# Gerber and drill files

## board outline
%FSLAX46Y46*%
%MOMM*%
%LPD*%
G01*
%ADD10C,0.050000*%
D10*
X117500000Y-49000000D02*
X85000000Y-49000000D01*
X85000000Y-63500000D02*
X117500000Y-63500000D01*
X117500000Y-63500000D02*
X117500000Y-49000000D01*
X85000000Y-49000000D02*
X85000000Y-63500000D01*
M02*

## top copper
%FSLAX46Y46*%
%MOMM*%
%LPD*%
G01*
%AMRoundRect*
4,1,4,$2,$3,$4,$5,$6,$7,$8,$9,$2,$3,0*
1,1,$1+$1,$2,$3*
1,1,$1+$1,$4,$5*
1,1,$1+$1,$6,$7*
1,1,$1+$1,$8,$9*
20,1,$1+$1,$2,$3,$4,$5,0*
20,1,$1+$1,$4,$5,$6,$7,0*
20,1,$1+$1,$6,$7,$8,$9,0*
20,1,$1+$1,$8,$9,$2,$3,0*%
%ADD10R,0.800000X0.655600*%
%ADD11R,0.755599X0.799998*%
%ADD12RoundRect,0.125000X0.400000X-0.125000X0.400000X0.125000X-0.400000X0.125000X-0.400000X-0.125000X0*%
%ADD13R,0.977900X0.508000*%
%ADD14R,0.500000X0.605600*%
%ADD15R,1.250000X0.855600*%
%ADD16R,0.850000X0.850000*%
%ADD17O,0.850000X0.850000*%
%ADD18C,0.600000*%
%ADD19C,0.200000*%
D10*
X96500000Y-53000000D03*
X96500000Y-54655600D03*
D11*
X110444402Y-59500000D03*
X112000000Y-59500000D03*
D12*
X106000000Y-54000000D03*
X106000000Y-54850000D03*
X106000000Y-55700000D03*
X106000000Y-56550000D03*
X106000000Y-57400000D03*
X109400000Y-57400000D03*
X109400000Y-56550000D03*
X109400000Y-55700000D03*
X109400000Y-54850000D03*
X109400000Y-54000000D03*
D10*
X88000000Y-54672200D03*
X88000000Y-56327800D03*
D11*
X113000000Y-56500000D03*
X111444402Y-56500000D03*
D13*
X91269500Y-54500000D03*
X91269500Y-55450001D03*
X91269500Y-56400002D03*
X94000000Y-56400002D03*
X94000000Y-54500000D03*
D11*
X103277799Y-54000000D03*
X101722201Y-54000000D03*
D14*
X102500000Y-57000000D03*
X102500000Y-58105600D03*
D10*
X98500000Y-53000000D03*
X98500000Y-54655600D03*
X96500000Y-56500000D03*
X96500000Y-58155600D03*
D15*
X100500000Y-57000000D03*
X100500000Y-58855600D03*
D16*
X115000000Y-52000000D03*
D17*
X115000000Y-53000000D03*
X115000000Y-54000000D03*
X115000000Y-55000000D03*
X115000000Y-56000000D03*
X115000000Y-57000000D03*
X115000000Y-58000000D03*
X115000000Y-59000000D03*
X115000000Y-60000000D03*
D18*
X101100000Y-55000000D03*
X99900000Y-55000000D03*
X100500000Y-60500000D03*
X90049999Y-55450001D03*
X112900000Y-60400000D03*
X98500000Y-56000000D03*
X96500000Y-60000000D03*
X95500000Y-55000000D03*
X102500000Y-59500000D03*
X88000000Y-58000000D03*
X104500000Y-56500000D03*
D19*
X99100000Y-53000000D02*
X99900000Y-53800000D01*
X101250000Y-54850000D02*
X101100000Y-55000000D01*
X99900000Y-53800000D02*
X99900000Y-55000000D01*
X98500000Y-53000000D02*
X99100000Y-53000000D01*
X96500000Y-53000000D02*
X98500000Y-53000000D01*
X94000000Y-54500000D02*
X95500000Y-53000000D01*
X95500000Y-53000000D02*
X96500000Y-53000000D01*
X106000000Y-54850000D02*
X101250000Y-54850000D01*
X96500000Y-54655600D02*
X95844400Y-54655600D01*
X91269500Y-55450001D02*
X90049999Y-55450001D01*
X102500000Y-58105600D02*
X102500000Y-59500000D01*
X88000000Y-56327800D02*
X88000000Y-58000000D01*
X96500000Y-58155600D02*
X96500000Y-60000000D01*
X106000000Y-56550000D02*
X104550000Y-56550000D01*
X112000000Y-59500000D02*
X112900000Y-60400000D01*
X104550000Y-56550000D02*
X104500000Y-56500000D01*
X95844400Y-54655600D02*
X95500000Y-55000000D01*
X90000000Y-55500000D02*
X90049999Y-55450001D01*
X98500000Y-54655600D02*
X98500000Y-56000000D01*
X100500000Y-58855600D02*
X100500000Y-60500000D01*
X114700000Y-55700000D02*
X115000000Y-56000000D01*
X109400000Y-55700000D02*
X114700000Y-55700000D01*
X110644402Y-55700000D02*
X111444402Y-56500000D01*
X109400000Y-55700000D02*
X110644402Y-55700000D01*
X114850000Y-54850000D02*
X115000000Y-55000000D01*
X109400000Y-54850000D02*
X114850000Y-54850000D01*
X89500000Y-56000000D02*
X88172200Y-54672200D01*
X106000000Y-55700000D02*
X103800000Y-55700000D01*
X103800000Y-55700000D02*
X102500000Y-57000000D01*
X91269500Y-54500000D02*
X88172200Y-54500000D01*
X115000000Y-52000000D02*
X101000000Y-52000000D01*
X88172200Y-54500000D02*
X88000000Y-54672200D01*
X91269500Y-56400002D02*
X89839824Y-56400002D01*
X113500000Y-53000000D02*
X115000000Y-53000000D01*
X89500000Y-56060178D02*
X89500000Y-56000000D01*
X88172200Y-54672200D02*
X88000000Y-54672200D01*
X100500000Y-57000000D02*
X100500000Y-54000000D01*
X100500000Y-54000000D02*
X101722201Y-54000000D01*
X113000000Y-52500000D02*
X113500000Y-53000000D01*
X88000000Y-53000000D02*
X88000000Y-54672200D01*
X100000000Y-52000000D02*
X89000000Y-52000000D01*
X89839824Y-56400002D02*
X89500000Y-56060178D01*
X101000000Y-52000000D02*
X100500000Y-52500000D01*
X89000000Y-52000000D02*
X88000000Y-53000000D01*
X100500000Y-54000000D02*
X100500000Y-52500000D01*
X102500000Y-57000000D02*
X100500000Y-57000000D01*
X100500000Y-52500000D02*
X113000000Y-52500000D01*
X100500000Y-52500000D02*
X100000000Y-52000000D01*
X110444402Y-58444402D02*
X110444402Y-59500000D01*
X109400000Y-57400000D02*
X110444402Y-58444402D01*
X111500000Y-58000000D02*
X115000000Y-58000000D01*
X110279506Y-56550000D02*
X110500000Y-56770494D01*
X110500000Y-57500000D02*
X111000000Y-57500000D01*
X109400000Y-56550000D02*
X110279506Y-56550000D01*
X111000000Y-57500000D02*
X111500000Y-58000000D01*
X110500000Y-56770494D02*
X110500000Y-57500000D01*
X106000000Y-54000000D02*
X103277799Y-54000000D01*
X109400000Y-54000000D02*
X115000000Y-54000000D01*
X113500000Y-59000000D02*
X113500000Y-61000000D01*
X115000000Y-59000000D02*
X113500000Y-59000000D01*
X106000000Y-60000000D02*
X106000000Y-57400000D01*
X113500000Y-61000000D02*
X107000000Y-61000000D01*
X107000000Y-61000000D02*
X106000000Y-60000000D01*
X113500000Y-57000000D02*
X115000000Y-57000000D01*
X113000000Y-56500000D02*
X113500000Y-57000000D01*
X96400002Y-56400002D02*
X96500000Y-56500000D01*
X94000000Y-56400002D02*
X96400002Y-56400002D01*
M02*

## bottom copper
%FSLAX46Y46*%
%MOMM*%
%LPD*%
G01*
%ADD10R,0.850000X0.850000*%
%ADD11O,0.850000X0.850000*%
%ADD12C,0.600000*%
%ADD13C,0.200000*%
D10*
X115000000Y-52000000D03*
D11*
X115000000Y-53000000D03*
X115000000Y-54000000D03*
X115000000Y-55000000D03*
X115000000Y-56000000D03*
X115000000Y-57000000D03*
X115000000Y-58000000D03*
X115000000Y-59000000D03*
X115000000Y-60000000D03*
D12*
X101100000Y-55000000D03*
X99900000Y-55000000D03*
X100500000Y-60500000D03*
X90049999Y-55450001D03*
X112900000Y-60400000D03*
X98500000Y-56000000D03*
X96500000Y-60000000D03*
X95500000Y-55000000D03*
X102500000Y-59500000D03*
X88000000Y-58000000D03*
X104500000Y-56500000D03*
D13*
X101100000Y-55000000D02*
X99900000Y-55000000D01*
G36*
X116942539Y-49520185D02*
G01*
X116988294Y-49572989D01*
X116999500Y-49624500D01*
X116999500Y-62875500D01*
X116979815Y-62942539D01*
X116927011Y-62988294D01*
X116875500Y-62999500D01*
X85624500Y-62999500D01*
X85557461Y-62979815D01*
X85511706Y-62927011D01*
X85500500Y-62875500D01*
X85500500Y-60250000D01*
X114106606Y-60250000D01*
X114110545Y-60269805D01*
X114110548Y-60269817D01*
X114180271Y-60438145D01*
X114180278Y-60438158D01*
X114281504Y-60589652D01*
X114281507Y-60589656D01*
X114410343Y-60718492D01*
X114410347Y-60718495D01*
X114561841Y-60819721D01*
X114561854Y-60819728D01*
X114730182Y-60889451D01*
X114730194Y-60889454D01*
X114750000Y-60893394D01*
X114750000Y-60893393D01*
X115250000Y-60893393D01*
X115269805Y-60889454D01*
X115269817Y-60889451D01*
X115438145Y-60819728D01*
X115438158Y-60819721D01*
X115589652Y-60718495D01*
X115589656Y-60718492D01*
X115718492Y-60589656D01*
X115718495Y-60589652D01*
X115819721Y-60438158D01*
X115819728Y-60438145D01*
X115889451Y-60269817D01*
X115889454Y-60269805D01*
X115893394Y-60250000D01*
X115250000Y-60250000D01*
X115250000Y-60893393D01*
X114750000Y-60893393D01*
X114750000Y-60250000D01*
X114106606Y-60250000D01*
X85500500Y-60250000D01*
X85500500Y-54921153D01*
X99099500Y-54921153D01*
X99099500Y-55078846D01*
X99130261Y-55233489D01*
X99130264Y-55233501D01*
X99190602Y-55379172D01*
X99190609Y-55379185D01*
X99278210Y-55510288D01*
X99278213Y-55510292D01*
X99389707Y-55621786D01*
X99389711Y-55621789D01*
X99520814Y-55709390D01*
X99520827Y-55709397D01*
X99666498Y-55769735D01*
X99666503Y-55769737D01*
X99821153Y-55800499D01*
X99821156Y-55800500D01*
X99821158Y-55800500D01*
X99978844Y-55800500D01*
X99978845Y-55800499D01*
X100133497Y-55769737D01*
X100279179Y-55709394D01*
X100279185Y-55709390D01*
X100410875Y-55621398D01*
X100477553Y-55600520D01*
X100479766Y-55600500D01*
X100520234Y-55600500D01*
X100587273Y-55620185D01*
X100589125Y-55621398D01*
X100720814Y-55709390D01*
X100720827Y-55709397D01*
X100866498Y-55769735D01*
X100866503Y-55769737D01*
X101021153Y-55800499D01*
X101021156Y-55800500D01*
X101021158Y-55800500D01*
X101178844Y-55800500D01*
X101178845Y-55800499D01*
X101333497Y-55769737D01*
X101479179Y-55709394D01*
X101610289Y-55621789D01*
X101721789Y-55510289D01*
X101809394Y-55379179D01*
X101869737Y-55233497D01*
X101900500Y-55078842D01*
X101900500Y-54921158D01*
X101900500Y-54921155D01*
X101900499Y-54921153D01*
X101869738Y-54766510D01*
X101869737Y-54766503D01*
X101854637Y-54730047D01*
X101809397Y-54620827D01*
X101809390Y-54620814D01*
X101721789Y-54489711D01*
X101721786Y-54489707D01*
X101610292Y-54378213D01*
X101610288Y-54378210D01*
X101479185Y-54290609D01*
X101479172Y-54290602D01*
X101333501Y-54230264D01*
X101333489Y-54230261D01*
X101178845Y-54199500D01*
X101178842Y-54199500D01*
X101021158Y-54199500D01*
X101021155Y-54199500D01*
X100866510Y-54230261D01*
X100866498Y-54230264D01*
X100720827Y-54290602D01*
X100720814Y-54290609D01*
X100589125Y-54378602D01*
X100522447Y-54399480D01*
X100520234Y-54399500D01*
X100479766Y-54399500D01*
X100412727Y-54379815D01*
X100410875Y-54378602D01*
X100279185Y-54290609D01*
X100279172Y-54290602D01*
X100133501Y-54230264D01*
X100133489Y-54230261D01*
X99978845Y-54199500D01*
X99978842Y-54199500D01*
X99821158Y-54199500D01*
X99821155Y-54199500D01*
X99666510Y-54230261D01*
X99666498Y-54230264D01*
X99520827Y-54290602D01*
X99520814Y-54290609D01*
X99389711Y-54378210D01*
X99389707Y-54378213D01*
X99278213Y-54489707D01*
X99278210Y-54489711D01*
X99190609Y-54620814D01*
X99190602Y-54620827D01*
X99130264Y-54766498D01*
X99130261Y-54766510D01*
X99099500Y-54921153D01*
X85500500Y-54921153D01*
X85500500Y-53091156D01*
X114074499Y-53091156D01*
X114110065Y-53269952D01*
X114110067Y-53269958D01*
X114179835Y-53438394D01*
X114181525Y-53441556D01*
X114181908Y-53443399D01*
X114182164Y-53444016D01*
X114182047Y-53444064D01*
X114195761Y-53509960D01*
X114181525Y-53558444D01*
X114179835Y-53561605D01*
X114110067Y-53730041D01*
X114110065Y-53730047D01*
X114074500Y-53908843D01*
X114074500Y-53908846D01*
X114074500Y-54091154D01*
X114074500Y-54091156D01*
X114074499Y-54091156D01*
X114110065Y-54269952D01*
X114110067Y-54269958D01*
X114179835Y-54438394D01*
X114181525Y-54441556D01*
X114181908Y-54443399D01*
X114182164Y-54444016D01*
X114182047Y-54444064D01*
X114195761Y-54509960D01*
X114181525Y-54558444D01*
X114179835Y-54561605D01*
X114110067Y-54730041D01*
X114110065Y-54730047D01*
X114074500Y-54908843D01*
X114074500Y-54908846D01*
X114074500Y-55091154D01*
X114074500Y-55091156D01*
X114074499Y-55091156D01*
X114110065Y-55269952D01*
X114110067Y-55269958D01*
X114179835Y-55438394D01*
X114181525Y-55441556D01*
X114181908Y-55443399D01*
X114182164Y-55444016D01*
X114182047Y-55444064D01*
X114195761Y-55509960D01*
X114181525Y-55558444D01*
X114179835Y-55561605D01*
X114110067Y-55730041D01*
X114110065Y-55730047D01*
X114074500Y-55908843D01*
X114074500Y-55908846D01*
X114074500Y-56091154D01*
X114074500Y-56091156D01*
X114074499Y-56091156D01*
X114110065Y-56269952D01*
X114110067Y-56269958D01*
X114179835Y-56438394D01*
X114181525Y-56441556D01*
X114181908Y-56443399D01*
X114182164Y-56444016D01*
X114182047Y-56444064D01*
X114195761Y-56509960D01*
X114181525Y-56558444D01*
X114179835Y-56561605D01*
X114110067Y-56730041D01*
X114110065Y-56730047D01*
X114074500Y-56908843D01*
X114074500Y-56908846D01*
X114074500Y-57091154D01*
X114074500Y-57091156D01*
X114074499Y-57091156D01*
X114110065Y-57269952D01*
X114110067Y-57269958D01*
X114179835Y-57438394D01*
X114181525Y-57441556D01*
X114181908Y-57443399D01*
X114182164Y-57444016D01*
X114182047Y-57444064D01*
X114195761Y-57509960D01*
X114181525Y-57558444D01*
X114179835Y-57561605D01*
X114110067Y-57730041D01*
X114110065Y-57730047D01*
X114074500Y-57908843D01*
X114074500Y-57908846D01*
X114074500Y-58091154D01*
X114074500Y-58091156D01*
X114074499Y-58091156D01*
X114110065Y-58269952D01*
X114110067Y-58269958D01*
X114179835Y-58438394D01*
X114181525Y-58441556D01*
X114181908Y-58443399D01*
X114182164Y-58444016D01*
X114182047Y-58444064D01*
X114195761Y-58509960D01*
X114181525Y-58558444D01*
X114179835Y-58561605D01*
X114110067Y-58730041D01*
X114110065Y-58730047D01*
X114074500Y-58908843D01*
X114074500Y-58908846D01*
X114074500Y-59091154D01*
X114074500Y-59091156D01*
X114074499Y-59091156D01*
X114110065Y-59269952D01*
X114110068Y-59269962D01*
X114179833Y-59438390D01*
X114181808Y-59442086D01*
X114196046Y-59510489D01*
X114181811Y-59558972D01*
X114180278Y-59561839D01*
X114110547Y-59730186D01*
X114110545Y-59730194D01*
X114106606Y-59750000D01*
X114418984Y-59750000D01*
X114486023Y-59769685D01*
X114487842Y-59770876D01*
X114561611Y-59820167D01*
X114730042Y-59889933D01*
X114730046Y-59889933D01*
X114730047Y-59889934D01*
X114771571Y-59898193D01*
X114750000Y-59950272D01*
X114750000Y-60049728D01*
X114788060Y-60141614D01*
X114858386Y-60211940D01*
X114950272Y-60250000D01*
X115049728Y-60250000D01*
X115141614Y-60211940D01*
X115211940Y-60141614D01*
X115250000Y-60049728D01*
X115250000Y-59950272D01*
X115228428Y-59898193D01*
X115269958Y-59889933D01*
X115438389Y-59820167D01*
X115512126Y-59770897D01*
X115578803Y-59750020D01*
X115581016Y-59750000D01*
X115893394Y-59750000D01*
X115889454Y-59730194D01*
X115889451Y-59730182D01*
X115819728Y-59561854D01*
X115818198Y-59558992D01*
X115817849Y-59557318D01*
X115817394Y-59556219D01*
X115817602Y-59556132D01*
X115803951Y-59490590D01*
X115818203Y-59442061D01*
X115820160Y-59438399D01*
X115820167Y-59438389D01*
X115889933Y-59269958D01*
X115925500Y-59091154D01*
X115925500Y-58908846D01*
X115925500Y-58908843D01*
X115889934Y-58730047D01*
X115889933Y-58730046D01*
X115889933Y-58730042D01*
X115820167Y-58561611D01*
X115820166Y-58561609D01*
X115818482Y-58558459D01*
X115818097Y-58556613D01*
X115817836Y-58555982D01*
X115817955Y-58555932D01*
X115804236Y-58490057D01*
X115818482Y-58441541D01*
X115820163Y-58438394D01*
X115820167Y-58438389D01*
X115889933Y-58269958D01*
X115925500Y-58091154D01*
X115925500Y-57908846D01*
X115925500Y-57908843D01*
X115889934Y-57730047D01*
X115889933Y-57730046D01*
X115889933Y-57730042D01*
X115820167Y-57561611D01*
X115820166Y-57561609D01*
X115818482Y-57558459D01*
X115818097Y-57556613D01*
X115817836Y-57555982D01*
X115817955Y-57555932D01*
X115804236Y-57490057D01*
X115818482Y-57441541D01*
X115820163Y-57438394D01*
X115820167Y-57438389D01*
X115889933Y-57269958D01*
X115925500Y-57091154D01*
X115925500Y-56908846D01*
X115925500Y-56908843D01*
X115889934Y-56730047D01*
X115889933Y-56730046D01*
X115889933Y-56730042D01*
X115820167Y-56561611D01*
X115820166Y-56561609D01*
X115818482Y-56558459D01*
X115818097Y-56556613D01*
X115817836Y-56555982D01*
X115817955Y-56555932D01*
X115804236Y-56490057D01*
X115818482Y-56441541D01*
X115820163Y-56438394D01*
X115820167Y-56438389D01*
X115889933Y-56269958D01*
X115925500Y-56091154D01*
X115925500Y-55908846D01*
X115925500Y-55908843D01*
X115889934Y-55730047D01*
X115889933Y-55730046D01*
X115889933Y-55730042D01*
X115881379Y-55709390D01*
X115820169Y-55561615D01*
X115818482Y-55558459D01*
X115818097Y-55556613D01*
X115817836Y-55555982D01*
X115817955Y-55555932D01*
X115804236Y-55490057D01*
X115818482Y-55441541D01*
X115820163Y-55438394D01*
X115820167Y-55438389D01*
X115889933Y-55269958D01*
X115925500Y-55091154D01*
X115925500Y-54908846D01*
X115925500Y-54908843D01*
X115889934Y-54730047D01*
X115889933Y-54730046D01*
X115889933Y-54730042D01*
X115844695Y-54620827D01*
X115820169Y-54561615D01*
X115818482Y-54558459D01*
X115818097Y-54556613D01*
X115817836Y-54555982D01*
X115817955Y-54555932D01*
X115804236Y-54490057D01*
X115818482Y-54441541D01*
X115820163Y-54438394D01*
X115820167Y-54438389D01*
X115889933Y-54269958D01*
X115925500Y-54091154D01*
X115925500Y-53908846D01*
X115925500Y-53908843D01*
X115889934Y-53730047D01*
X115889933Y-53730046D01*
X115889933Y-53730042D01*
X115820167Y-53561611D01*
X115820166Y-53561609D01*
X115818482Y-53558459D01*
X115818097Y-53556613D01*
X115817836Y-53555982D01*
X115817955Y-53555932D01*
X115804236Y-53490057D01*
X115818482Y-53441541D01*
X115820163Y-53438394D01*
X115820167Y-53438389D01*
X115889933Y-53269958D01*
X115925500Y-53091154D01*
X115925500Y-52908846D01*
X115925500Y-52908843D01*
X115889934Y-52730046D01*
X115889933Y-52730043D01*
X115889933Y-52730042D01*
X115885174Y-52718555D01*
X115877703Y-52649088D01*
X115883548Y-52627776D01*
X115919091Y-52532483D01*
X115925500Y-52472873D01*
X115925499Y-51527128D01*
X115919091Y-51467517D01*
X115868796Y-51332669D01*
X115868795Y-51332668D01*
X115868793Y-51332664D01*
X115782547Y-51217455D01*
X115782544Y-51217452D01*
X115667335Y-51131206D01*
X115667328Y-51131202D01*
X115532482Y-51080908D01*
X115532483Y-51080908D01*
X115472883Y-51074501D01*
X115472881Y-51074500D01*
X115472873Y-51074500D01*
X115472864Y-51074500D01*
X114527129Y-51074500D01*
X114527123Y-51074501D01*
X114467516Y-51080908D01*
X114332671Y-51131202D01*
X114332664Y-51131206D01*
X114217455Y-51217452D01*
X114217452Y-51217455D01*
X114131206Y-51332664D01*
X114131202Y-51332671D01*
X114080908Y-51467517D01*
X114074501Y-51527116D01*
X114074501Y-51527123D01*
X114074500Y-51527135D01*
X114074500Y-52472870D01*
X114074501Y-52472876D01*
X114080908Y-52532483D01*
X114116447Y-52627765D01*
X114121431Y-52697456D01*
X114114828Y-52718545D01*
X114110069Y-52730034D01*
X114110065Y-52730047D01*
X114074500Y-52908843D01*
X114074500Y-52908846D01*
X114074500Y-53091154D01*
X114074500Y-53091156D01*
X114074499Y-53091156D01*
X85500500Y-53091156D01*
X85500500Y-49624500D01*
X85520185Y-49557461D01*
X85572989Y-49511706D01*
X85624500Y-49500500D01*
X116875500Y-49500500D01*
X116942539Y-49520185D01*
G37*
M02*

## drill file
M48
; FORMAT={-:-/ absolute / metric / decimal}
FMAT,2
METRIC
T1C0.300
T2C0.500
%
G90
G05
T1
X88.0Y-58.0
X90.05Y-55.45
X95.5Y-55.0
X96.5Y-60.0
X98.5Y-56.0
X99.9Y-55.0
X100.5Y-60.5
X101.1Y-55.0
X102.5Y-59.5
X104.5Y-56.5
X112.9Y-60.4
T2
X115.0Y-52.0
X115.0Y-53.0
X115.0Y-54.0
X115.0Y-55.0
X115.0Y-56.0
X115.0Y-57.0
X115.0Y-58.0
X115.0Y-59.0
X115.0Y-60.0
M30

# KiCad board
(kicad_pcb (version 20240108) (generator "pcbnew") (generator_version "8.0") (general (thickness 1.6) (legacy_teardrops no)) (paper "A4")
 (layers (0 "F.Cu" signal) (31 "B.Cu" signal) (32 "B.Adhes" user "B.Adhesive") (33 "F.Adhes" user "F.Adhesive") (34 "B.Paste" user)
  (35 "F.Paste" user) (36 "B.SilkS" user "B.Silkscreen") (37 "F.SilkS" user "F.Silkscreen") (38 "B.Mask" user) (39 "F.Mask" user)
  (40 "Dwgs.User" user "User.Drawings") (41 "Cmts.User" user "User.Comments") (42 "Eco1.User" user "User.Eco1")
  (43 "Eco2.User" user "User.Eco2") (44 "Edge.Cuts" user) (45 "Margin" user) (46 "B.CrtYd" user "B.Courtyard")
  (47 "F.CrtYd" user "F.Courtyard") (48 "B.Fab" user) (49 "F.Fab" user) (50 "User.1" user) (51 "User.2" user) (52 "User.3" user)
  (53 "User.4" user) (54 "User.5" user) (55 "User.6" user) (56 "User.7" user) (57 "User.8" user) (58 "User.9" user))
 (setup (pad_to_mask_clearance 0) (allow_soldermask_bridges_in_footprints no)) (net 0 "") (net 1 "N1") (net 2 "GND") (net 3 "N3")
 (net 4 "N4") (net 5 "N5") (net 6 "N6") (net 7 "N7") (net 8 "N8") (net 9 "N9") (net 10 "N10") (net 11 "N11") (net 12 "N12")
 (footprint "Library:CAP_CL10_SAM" (layer "F.Cu") (at 96.5 53.8278 -90)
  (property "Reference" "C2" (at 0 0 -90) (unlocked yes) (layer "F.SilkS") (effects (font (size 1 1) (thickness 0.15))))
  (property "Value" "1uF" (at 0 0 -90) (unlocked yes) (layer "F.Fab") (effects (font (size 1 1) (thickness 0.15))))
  (pad "1" smd rect (at -0.8278 0 270) (size 0.6556 0.8) (layers "F.Cu" "F.Paste" "F.Mask") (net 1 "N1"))
  (pad "2" smd rect (at 0.8278 0 270) (size 0.6556 0.8) (layers "F.Cu" "F.Paste" "F.Mask") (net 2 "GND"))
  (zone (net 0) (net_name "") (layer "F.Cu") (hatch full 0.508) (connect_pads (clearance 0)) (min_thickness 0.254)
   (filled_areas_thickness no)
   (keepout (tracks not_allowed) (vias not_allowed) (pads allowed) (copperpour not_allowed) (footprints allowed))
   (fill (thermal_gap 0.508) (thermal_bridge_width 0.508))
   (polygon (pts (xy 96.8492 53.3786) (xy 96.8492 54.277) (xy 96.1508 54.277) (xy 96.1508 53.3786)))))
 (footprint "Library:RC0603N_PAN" (layer "F.Cu") (at 111.222201 59.5)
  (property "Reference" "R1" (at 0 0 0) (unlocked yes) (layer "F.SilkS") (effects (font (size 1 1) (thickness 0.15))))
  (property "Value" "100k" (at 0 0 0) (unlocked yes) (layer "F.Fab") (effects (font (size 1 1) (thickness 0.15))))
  (pad "1" smd rect (at -0.777799 0) (size 0.755599 0.799998) (layers "F.Cu" "F.Paste" "F.Mask") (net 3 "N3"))
  (pad "2" smd rect (at 0.777799 0) (size 0.755599 0.799998) (layers "F.Cu" "F.Paste" "F.Mask") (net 2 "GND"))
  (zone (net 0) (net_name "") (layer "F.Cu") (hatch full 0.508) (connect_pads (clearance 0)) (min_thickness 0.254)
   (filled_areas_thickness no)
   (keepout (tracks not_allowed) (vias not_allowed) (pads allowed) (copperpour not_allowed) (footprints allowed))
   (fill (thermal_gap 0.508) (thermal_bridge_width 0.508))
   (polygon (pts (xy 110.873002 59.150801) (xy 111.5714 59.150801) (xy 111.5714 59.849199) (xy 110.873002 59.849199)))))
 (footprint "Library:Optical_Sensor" (layer "F.Cu") (at 116.5 60.5)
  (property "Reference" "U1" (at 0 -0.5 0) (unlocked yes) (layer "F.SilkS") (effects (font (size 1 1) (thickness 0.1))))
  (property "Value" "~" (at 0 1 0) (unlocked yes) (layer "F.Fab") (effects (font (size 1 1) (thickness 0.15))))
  (pad "1" smd roundrect (at -10.5 -6.5 90) (size 0.5 1.05) (layers "F.Cu" "F.Paste" "F.Mask") (roundrect_rratio 0.25) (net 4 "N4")
   (thermal_bridge_angle 45))
  (pad "2" smd roundrect (at -10.5 -5.65 90) (size 0.5 1.05) (layers "F.Cu" "F.Paste" "F.Mask") (roundrect_rratio 0.25) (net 1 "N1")
   (thermal_bridge_angle 45))
  (pad "3" smd roundrect (at -10.5 -4.8 90) (size 0.5 1.05) (layers "F.Cu" "F.Paste" "F.Mask") (roundrect_rratio 0.25) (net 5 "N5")
   (thermal_bridge_angle 45))
  (pad "4" smd roundrect (at -10.5 -3.95 90) (size 0.5 1.05) (layers "F.Cu" "F.Paste" "F.Mask") (roundrect_rratio 0.25) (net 2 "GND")
   (thermal_bridge_angle 45))
  (pad "5" smd roundrect (at -10.5 -3.1 90) (size 0.5 1.05) (layers "F.Cu" "F.Paste" "F.Mask") (roundrect_rratio 0.25) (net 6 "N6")
   (thermal_bridge_angle 45))
  (pad "6" smd roundrect (at -7.1 -3.1 90) (size 0.5 1.05) (layers "F.Cu" "F.Paste" "F.Mask") (roundrect_rratio 0.25) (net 3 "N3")
   (thermal_bridge_angle 45))
  (pad "7" smd roundrect (at -7.1 -3.95 90) (size 0.5 1.05) (layers "F.Cu" "F.Paste" "F.Mask") (roundrect_rratio 0.25) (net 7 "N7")
   (thermal_bridge_angle 45))
  (pad "8" smd roundrect (at -7.1 -4.8 90) (size 0.5 1.05) (layers "F.Cu" "F.Paste" "F.Mask") (roundrect_rratio 0.25) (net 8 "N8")
   (thermal_bridge_angle 45))
  (pad "9" smd roundrect (at -7.1 -5.65 90) (size 0.5 1.05) (layers "F.Cu" "F.Paste" "F.Mask") (roundrect_rratio 0.25) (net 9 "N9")
   (thermal_bridge_angle 45))
  (pad "10" smd roundrect (at -7.1 -6.5 90) (size 0.5 1.05) (layers "F.Cu" "F.Paste" "F.Mask") (roundrect_rratio 0.25) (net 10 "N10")
   (thermal_bridge_angle 45)))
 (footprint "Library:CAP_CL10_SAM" (layer "F.Cu") (at 88 55.5 -90)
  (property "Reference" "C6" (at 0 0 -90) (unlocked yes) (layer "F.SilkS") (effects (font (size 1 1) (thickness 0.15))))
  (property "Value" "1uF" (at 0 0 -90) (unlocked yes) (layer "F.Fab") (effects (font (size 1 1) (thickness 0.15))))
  (pad "1" smd rect (at -0.8278 0 270) (size 0.6556 0.8) (layers "F.Cu" "F.Paste" "F.Mask") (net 5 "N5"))
  (pad "2" smd rect (at 0.8278 0 270) (size 0.6556 0.8) (layers "F.Cu" "F.Paste" "F.Mask") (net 2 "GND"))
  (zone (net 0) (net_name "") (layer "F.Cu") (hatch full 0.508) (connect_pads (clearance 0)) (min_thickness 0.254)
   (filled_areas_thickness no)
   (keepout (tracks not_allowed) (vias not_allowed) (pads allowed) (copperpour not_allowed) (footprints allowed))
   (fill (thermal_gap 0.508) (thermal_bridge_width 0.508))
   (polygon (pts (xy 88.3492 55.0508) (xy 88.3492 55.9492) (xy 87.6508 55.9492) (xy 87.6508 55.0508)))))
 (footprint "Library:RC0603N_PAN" (layer "F.Cu") (at 112.222201 56.5 180)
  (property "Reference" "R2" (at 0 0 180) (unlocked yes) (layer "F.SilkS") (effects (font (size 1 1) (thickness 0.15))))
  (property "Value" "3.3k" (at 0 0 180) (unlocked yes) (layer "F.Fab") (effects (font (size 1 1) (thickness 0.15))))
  (pad "1" smd rect (at -0.777799 0 180) (size 0.755599 0.799998) (layers "F.Cu" "F.Paste" "F.Mask") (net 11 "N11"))
  (pad "2" smd rect (at 0.777799 0 180) (size 0.755599 0.799998) (layers "F.Cu" "F.Paste" "F.Mask") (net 8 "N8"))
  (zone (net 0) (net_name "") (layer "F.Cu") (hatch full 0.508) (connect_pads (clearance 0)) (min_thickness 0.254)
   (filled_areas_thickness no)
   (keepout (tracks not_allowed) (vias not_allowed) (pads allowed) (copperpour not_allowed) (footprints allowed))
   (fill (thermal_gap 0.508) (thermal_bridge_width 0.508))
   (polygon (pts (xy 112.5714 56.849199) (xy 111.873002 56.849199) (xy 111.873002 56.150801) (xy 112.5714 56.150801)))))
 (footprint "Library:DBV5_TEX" (layer "F.Cu") (at 92.63475 55.450001)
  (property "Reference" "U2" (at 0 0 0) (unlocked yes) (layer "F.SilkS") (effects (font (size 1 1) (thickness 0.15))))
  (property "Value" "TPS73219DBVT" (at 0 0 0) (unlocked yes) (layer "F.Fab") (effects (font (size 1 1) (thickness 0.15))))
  (pad "1" smd rect (at -1.36525 -0.950001) (size 0.9779 0.508) (layers "F.Cu" "F.Paste" "F.Mask") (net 5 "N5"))
  (pad "2" smd rect (at -1.36525 0) (size 0.9779 0.508) (layers "F.Cu" "F.Paste" "F.Mask") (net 2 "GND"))
  (pad "3" smd rect (at -1.36525 0.950001) (size 0.9779 0.508) (layers "F.Cu" "F.Paste" "F.Mask") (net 5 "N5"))
  (pad "4" smd rect (at 1.36525 0.950001) (size 0.9779 0.508) (layers "F.Cu" "F.Paste" "F.Mask") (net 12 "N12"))
  (pad "5" smd rect (at 1.36525 -0.950001) (size 0.9779 0.508) (layers "F.Cu" "F.Paste" "F.Mask") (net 1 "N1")))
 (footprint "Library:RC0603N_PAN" (layer "F.Cu") (at 102.5 54 180)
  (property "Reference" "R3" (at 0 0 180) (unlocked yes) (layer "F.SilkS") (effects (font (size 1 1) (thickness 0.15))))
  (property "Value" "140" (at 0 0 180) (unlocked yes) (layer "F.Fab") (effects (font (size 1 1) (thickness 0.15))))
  (pad "1" smd rect (at -0.777799 0 180) (size 0.755599 0.799998) (layers "F.Cu" "F.Paste" "F.Mask") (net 4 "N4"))
  (pad "2" smd rect (at 0.777799 0 180) (size 0.755599 0.799998) (layers "F.Cu" "F.Paste" "F.Mask") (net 5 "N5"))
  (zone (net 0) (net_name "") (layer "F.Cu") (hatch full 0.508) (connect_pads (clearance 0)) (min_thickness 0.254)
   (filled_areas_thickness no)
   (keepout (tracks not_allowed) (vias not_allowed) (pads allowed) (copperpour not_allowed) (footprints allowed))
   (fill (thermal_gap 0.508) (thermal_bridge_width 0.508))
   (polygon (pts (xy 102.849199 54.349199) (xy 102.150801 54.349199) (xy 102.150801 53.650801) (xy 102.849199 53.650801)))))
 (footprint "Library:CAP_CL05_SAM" (layer "F.Cu") (at 102.5 57.5528 -90)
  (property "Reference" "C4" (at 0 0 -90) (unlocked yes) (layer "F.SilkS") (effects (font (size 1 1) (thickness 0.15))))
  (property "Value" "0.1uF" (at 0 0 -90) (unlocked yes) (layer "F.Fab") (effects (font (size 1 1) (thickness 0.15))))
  (pad "1" smd rect (at -0.5528 0 270) (size 0.6056 0.5) (layers "F.Cu" "F.Paste" "F.Mask") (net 5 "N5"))
  (pad "2" smd rect (at 0.5528 0 270) (size 0.6056 0.5) (layers "F.Cu" "F.Paste" "F.Mask") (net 2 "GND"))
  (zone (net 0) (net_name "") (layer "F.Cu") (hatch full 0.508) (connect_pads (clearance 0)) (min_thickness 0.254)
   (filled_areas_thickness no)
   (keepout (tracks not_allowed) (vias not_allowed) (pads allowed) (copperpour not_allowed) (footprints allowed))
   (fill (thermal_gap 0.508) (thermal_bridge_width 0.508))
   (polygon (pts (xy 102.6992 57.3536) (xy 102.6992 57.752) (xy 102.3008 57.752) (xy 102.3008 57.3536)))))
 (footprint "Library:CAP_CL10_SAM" (layer "F.Cu") (at 98.5 53.8278 -90)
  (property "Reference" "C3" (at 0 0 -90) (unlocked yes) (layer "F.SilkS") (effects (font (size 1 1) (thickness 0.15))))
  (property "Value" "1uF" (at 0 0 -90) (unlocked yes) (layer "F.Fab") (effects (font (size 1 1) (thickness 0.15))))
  (pad "1" smd rect (at -0.8278 0 270) (size 0.6556 0.8) (layers "F.Cu" "F.Paste" "F.Mask") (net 1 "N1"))
  (pad "2" smd rect (at 0.8278 0 270) (size 0.6556 0.8) (layers "F.Cu" "F.Paste" "F.Mask") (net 2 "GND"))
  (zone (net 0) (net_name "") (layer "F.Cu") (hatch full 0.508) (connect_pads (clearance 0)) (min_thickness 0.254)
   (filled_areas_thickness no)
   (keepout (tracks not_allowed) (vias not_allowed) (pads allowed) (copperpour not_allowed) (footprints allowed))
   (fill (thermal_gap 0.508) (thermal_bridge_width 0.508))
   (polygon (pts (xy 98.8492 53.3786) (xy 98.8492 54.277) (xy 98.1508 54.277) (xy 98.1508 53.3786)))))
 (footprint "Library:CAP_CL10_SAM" (layer "F.Cu") (at 96.5 57.3278 -90)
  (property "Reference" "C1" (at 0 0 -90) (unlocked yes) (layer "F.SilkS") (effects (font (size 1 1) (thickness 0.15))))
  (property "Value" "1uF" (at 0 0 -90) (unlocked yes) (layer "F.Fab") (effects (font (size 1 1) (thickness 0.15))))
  (pad "1" smd rect (at -0.8278 0 270) (size 0.6556 0.8) (layers "F.Cu" "F.Paste" "F.Mask") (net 12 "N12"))
  (pad "2" smd rect (at 0.8278 0 270) (size 0.6556 0.8) (layers "F.Cu" "F.Paste" "F.Mask") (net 2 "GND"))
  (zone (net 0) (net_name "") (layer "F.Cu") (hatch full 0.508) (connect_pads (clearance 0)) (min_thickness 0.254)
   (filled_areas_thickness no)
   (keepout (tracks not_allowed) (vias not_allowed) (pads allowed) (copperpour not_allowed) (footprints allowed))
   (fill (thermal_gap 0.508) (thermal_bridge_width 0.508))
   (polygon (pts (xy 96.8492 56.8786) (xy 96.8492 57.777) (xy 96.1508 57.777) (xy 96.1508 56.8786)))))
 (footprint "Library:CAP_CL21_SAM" (layer "F.Cu") (at 100.5 57.9278 -90)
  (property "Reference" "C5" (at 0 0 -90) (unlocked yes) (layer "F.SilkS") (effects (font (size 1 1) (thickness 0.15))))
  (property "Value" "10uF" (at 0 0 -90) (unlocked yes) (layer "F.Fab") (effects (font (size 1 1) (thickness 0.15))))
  (pad "1" smd rect (at -0.9278 0 270) (size 0.8556 1.25) (layers "F.Cu" "F.Paste" "F.Mask") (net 5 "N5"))
  (pad "2" smd rect (at 0.9278 0 270) (size 0.8556 1.25) (layers "F.Cu" "F.Paste" "F.Mask") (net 2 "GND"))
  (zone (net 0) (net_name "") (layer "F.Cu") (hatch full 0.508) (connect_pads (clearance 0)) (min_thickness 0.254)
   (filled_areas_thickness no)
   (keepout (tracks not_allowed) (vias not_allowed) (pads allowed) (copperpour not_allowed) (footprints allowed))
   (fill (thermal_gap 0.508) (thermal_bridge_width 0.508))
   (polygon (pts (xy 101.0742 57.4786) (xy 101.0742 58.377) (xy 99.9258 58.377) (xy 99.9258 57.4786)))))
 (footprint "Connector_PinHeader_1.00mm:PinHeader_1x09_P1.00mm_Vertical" (layer "F.Cu") (at 115 52)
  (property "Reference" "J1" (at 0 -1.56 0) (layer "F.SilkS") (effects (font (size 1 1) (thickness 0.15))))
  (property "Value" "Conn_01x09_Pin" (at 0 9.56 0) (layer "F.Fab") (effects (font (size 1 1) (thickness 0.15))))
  (pad "1" thru_hole rect (at 0 0) (size 0.85 0.85) (drill 0.5) (layers "*.Cu" "*.Mask") (remove_unused_layers no) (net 5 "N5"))
  (pad "2" thru_hole oval (at 0 1) (size 0.85 0.85) (drill 0.5) (layers "*.Cu" "*.Mask") (remove_unused_layers no) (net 5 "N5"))
  (pad "3" thru_hole oval (at 0 2) (size 0.85 0.85) (drill 0.5) (layers "*.Cu" "*.Mask") (remove_unused_layers no) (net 10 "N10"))
  (pad "4" thru_hole oval (at 0 3) (size 0.85 0.85) (drill 0.5) (layers "*.Cu" "*.Mask") (remove_unused_layers no) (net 9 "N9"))
  (pad "5" thru_hole oval (at 0 4) (size 0.85 0.85) (drill 0.5) (layers "*.Cu" "*.Mask") (remove_unused_layers no) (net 8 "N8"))
  (pad "6" thru_hole oval (at 0 5) (size 0.85 0.85) (drill 0.5) (layers "*.Cu" "*.Mask") (remove_unused_layers no) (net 11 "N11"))
  (pad "7" thru_hole oval (at 0 6) (size 0.85 0.85) (drill 0.5) (layers "*.Cu" "*.Mask") (remove_unused_layers no) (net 7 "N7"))
  (pad "8" thru_hole oval (at 0 7) (size 0.85 0.85) (drill 0.5) (layers "*.Cu" "*.Mask") (remove_unused_layers no) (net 6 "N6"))
  (pad "9" thru_hole oval (at 0 8) (size 0.85 0.85) (drill 0.5) (layers "*.Cu" "*.Mask") (remove_unused_layers no) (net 2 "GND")))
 (gr_line (start 117.5 49) (end 85 49) (stroke (width 0.05) (type default)) (layer "Edge.Cuts"))
 (gr_line (start 85 63.5) (end 117.5 63.5) (stroke (width 0.05) (type default)) (layer "Edge.Cuts"))
 (gr_line (start 117.5 63.5) (end 117.5 49) (stroke (width 0.05) (type default)) (layer "Edge.Cuts"))
 (gr_line (start 85 49) (end 85 63.5) (stroke (width 0.05) (type default)) (layer "Edge.Cuts"))
 (segment (start 99.1 53) (end 99.9 53.8) (width 0.2) (layer "F.Cu") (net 1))
 (segment (start 101.25 54.85) (end 101.1 55) (width 0.2) (layer "F.Cu") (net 1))
 (segment (start 99.9 53.8) (end 99.9 55) (width 0.2) (layer "F.Cu") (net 1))
 (segment (start 98.5 53) (end 99.1 53) (width 0.2) (layer "F.Cu") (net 1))
 (segment (start 96.5 53) (end 98.5 53) (width 0.2) (layer "F.Cu") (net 1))
 (segment (start 94 54.5) (end 95.5 53) (width 0.2) (layer "F.Cu") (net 1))
 (segment (start 95.5 53) (end 96.5 53) (width 0.2) (layer "F.Cu") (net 1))
 (segment (start 106 54.85) (end 101.25 54.85) (width 0.2) (layer "F.Cu") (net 1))
 (via (at 101.1 55) (size 0.6) (drill 0.3) (layers "F.Cu" "B.Cu") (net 1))
 (via (at 99.9 55) (size 0.6) (drill 0.3) (layers "F.Cu" "B.Cu") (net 1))
 (segment (start 101.1 55) (end 99.9 55) (width 0.2) (layer "B.Cu") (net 1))
 (segment (start 96.5 54.6556) (end 95.8444 54.6556) (width 0.2) (layer "F.Cu") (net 2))
 (segment (start 91.2695 55.450001) (end 90.049999 55.450001) (width 0.2) (layer "F.Cu") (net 2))
 (segment (start 102.5 58.1056) (end 102.5 59.5) (width 0.2) (layer "F.Cu") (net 2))
 (segment (start 88 56.3278) (end 88 58) (width 0.2) (layer "F.Cu") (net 2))
 (segment (start 96.5 58.1556) (end 96.5 60) (width 0.2) (layer "F.Cu") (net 2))
 (segment (start 106 56.55) (end 104.55 56.55) (width 0.2) (layer "F.Cu") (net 2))
 (segment (start 112 59.5) (end 112.9 60.4) (width 0.2) (layer "F.Cu") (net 2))
 (segment (start 104.55 56.55) (end 104.5 56.5) (width 0.2) (layer "F.Cu") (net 2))
 (segment (start 95.8444 54.6556) (end 95.5 55) (width 0.2) (layer "F.Cu") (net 2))
 (segment (start 90 55.5) (end 90.049999 55.450001) (width 0.2) (layer "F.Cu") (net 2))
 (segment (start 98.5 54.6556) (end 98.5 56) (width 0.2) (layer "F.Cu") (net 2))
 (segment (start 100.5 58.8556) (end 100.5 60.5) (width 0.2) (layer "F.Cu") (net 2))
 (via (at 100.5 60.5) (size 0.6) (drill 0.3) (layers "F.Cu" "B.Cu") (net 2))
 (via (at 90.049999 55.450001) (size 0.6) (drill 0.3) (layers "F.Cu" "B.Cu") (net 2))
 (via (at 112.9 60.4) (size 0.6) (drill 0.3) (layers "F.Cu" "B.Cu") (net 2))
 (via (at 98.5 56) (size 0.6) (drill 0.3) (layers "F.Cu" "B.Cu") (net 2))
 (via (at 96.5 60) (size 0.6) (drill 0.3) (layers "F.Cu" "B.Cu") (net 2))
 (via (at 95.5 55) (size 0.6) (drill 0.3) (layers "F.Cu" "B.Cu") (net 2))
 (via (at 102.5 59.5) (size 0.6) (drill 0.3) (layers "F.Cu" "B.Cu") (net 2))
 (via (at 88 58) (size 0.6) (drill 0.3) (layers "F.Cu" "B.Cu") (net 2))
 (via (at 104.5 56.5) (size 0.6) (drill 0.3) (layers "F.Cu" "B.Cu") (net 2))
 (segment (start 114.7 55.7) (end 115 56) (width 0.2) (layer "F.Cu") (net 8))
 (segment (start 109.4 55.7) (end 114.7 55.7) (width 0.2) (layer "F.Cu") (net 8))
 (segment (start 110.644402 55.7) (end 111.444402 56.5) (width 0.2) (layer "F.Cu") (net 8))
 (segment (start 109.4 55.7) (end 110.644402 55.7) (width 0.2) (layer "F.Cu") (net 8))
 (segment (start 114.85 54.85) (end 115 55) (width 0.2) (layer "F.Cu") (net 9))
 (segment (start 109.4 54.85) (end 114.85 54.85) (width 0.2) (layer "F.Cu") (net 9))
 (segment (start 89.5 56) (end 88.1722 54.6722) (width 0.2) (layer "F.Cu") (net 5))
 (segment (start 106 55.7) (end 103.8 55.7) (width 0.2) (layer "F.Cu") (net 5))
 (segment (start 103.8 55.7) (end 102.5 57) (width 0.2) (layer "F.Cu") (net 5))
 (segment (start 91.2695 54.5) (end 88.1722 54.5) (width 0.2) (layer "F.Cu") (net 5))
 (segment (start 115 52) (end 101 52) (width 0.2) (layer "F.Cu") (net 5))
 (segment (start 88.1722 54.5) (end 88 54.6722) (width 0.2) (layer "F.Cu") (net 5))
 (segment (start 91.2695 56.400002) (end 89.839824 56.400002) (width 0.2) (layer "F.Cu") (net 5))
 (segment (start 113.5 53) (end 115 53) (width 0.2) (layer "F.Cu") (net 5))
 (segment (start 89.5 56.060178) (end 89.5 56) (width 0.2) (layer "F.Cu") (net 5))
 (segment (start 88.1722 54.6722) (end 88 54.6722) (width 0.2) (layer "F.Cu") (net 5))
 (segment (start 100.5 57) (end 100.5 54) (width 0.2) (layer "F.Cu") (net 5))
 (segment (start 100.5 54) (end 101.722201 54) (width 0.2) (layer "F.Cu") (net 5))
 (segment (start 113 52.5) (end 113.5 53) (width 0.2) (layer "F.Cu") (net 5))
 (segment (start 88 53) (end 88 54.6722) (width 0.2) (layer "F.Cu") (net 5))
 (segment (start 100 52) (end 89 52) (width 0.2) (layer "F.Cu") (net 5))
 (segment (start 89.839824 56.400002) (end 89.5 56.060178) (width 0.2) (layer "F.Cu") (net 5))
 (segment (start 101 52) (end 100.5 52.5) (width 0.2) (layer "F.Cu") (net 5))
 (segment (start 89 52) (end 88 53) (width 0.2) (layer "F.Cu") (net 5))
 (segment (start 100.5 54) (end 100.5 52.5) (width 0.2) (layer "F.Cu") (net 5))
 (segment (start 102.5 57) (end 100.5 57) (width 0.2) (layer "F.Cu") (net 5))
 (segment (start 100.5 52.5) (end 113 52.5) (width 0.2) (layer "F.Cu") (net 5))
 (segment (start 100.5 52.5) (end 100 52) (width 0.2) (layer "F.Cu") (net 5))
 (segment (start 110.444402 58.444402) (end 110.444402 59.5) (width 0.2) (layer "F.Cu") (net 3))
 (segment (start 109.4 57.4) (end 110.444402 58.444402) (width 0.2) (layer "F.Cu") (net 3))
 (segment (start 111.5 58) (end 115 58) (width 0.2) (layer "F.Cu") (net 7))
 (segment (start 110.279506 56.55) (end 110.5 56.770494) (width 0.2) (layer "F.Cu") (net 7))
 (segment (start 110.5 57.5) (end 111 57.5) (width 0.2) (layer "F.Cu") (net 7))
 (segment (start 109.4 56.55) (end 110.279506 56.55) (width 0.2) (layer "F.Cu") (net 7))
 (segment (start 111 57.5) (end 111.5 58) (width 0.2) (layer "F.Cu") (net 7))
 (segment (start 110.5 56.770494) (end 110.5 57.5) (width 0.2) (layer "F.Cu") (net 7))
 (segment (start 106 54) (end 103.277799 54) (width 0.2) (layer "F.Cu") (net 4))
 (segment (start 109.4 54) (end 115 54) (width 0.2) (layer "F.Cu") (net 10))
 (segment (start 113.5 59) (end 113.5 61) (width 0.2) (layer "F.Cu") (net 6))
 (segment (start 115 59) (end 113.5 59) (width 0.2) (layer "F.Cu") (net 6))
 (segment (start 106 60) (end 106 57.4) (width 0.2) (layer "F.Cu") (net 6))
 (segment (start 113.5 61) (end 107 61) (width 0.2) (layer "F.Cu") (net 6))
 (segment (start 107 61) (end 106 60) (width 0.2) (layer "F.Cu") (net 6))
 (segment (start 113.5 57) (end 115 57) (width 0.2) (layer "F.Cu") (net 11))
 (segment (start 113 56.5) (end 113.5 57) (width 0.2) (layer "F.Cu") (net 11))
 (segment (start 96.400002 56.400002) (end 96.5 56.5) (width 0.2) (layer "F.Cu") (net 12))
 (segment (start 94 56.400002) (end 96.400002 56.400002) (width 0.2) (layer "F.Cu") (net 12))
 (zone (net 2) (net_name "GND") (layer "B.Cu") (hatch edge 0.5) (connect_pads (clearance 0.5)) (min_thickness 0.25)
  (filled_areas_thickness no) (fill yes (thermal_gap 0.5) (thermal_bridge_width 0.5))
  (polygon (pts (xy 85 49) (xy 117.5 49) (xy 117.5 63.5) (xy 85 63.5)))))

